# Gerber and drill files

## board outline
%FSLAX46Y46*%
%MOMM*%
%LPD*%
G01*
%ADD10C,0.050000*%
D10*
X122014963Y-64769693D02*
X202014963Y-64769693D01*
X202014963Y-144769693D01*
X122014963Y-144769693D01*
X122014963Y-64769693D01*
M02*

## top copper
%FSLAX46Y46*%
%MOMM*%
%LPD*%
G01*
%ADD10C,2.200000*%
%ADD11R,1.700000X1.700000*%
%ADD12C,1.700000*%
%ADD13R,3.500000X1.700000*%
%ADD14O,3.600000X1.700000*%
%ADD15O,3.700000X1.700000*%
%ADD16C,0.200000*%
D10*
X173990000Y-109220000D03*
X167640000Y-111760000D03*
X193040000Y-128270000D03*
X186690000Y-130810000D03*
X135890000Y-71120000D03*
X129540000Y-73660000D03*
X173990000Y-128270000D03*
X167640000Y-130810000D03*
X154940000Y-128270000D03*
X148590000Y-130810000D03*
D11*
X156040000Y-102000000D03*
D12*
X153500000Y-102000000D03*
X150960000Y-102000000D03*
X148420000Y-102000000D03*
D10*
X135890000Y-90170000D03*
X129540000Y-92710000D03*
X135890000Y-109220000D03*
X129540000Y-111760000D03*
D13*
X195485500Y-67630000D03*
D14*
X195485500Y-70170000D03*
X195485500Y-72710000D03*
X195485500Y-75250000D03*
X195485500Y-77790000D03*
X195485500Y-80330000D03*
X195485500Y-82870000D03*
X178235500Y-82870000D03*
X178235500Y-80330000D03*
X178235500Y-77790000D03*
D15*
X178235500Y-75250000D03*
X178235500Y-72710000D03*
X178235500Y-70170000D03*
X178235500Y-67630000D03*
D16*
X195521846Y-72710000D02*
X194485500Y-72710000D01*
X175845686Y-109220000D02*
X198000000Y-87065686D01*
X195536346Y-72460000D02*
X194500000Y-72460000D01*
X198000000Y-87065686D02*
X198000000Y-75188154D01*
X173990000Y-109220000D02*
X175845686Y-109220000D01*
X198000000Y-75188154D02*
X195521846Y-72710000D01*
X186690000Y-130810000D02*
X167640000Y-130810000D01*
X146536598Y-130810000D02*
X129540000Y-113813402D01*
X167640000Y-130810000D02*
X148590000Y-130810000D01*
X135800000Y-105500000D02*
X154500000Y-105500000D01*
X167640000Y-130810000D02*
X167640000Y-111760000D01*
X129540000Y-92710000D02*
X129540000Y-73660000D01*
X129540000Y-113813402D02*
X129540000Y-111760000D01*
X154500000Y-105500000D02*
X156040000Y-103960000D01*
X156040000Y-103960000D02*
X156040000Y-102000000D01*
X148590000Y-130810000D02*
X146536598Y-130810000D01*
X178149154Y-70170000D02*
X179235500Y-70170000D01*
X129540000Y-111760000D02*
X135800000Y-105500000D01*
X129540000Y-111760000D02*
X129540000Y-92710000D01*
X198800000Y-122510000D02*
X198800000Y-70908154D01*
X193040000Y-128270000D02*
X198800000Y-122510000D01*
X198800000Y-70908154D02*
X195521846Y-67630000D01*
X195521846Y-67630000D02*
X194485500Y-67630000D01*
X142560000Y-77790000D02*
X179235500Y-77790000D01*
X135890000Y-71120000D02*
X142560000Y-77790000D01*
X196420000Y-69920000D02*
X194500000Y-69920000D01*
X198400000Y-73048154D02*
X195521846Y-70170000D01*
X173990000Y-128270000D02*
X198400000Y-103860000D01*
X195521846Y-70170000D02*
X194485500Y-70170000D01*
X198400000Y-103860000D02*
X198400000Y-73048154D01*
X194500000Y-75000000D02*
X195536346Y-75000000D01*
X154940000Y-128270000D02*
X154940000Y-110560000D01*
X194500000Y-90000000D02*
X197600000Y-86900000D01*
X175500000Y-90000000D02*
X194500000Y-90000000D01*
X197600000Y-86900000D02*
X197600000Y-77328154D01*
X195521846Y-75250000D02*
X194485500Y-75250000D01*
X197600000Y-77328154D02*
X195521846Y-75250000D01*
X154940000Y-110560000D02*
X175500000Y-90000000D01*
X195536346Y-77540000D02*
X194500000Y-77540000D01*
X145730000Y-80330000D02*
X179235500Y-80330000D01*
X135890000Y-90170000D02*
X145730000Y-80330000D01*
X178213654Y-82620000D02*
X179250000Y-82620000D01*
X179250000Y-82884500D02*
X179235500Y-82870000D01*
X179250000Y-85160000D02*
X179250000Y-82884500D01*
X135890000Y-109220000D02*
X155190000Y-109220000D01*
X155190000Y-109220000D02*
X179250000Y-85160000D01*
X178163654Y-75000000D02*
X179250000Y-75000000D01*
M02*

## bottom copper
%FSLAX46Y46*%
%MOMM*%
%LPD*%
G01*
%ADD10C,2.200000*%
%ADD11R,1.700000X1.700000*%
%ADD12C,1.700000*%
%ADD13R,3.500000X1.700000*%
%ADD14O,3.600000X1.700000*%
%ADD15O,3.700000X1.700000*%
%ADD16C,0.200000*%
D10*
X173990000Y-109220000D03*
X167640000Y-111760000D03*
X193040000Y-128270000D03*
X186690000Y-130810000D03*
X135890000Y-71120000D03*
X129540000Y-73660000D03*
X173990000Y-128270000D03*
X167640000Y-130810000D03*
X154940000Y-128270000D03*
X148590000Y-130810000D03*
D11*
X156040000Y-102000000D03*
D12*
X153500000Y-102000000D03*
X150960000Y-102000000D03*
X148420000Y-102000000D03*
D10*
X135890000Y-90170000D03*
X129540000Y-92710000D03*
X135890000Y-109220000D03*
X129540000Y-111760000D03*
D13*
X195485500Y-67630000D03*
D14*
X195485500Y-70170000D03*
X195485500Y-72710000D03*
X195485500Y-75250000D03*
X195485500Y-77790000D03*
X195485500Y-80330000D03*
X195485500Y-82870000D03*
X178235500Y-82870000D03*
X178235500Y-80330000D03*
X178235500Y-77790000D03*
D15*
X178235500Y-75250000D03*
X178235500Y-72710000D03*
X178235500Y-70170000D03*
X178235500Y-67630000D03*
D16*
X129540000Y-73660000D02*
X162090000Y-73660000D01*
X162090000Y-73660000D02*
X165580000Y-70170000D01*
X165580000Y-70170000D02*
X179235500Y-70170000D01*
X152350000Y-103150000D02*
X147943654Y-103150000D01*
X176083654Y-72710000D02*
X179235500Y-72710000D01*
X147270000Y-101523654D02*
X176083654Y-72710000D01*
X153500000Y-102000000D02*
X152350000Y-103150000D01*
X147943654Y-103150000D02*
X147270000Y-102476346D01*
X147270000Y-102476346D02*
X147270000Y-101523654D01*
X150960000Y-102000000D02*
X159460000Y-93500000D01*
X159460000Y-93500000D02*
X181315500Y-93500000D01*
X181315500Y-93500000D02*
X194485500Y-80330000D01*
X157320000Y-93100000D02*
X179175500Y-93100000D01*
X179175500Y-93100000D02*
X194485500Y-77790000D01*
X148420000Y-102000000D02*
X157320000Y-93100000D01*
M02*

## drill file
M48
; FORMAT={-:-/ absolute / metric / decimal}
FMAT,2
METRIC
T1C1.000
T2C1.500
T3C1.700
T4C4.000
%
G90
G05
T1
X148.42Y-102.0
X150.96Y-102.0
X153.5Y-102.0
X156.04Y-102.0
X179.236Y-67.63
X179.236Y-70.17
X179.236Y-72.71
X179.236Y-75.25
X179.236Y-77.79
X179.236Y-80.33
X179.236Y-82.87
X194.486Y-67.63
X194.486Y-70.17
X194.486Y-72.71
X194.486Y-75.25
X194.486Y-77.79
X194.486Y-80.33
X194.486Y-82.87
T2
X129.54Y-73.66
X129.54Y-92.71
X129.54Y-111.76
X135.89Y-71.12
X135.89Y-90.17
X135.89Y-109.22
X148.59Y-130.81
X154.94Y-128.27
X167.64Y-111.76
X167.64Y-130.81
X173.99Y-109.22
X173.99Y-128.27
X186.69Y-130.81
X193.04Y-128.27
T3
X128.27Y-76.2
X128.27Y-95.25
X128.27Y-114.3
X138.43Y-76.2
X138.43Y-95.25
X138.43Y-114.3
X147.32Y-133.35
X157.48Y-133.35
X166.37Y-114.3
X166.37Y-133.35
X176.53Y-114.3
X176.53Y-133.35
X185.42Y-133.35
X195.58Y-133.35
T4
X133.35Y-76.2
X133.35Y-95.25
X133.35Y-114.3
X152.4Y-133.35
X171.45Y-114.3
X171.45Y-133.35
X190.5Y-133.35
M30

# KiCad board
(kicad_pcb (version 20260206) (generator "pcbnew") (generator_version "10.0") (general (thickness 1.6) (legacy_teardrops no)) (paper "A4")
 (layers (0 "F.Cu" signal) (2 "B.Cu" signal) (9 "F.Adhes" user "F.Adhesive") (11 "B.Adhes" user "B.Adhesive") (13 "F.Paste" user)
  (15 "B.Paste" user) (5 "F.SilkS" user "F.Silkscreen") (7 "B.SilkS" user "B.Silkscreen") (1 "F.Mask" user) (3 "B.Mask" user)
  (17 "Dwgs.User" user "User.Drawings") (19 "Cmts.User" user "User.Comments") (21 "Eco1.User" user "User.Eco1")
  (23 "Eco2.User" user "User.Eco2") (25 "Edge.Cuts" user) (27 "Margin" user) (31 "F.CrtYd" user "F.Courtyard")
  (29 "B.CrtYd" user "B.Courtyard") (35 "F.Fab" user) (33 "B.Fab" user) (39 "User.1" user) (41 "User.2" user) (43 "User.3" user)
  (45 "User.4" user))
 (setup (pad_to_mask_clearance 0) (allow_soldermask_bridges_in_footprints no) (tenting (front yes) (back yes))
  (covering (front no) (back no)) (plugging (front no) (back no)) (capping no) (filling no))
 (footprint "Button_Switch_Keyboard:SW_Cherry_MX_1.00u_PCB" (layer "F.Cu") (at 173.99 109.22)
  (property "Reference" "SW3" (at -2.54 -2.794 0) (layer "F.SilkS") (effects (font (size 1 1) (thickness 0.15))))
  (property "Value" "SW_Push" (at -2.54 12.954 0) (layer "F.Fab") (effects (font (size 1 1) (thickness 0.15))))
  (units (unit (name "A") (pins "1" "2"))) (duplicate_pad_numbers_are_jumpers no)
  (pad "" np_thru_hole circle (at -7.62 5.08) (size 1.7 1.7) (drill 1.7) (layers "*.Cu" "*.Mask"))
  (pad "" np_thru_hole circle (at -2.54 5.08) (size 4 4) (drill 4) (layers "*.Cu" "*.Mask"))
  (pad "" np_thru_hole circle (at 2.54 5.08) (size 1.7 1.7) (drill 1.7) (layers "*.Cu" "*.Mask"))
  (pad "1" thru_hole circle (at 0 0) (size 2.2 2.2) (drill 1.5) (layers "*.Cu" "*.Mask") (remove_unused_layers no)
   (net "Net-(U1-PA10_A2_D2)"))
  (pad "2" thru_hole circle (at -6.35 2.54) (size 2.2 2.2) (drill 1.5) (layers "*.Cu" "*.Mask") (remove_unused_layers no) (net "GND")))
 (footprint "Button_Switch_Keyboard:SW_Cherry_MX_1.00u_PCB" (layer "F.Cu") (at 193.04 128.27)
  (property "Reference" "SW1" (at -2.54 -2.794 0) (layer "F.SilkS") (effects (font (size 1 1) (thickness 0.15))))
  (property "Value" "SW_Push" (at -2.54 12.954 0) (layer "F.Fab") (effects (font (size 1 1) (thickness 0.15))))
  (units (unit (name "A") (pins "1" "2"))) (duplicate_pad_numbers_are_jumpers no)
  (pad "" np_thru_hole circle (at -7.62 5.08) (size 1.7 1.7) (drill 1.7) (layers "*.Cu" "*.Mask"))
  (pad "" np_thru_hole circle (at -2.54 5.08) (size 4 4) (drill 4) (layers "*.Cu" "*.Mask"))
  (pad "" np_thru_hole circle (at 2.54 5.08) (size 1.7 1.7) (drill 1.7) (layers "*.Cu" "*.Mask"))
  (pad "1" thru_hole circle (at 0 0) (size 2.2 2.2) (drill 1.5) (layers "*.Cu" "*.Mask") (remove_unused_layers no)
   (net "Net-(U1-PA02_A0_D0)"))
  (pad "2" thru_hole circle (at -6.35 2.54) (size 2.2 2.2) (drill 1.5) (layers "*.Cu" "*.Mask") (remove_unused_layers no) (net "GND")))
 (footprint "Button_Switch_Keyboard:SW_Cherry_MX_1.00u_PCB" (layer "F.Cu") (at 135.89 71.12)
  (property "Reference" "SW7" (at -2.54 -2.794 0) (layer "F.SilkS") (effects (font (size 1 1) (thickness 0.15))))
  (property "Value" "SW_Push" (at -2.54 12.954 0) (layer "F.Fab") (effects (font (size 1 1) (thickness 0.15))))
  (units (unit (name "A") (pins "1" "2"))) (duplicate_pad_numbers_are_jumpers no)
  (pad "" np_thru_hole circle (at -7.62 5.08) (size 1.7 1.7) (drill 1.7) (layers "*.Cu" "*.Mask"))
  (pad "" np_thru_hole circle (at -2.54 5.08) (size 4 4) (drill 4) (layers "*.Cu" "*.Mask"))
  (pad "" np_thru_hole circle (at 2.54 5.08) (size 1.7 1.7) (drill 1.7) (layers "*.Cu" "*.Mask"))
  (pad "1" thru_hole circle (at 0 0) (size 2.2 2.2) (drill 1.5) (layers "*.Cu" "*.Mask") (remove_unused_layers no)
   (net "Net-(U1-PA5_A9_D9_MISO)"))
  (pad "2" thru_hole circle (at -6.35 2.54) (size 2.2 2.2) (drill 1.5) (layers "*.Cu" "*.Mask") (remove_unused_layers no) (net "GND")))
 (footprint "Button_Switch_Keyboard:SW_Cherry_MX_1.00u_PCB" (layer "F.Cu") (at 173.99 128.27)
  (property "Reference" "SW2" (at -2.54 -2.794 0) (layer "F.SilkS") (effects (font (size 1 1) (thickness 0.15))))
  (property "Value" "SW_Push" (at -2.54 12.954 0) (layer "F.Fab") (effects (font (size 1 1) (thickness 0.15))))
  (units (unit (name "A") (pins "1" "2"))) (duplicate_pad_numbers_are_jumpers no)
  (pad "" np_thru_hole circle (at -7.62 5.08) (size 1.7 1.7) (drill 1.7) (layers "*.Cu" "*.Mask"))
  (pad "" np_thru_hole circle (at -2.54 5.08) (size 4 4) (drill 4) (layers "*.Cu" "*.Mask"))
  (pad "" np_thru_hole circle (at 2.54 5.08) (size 1.7 1.7) (drill 1.7) (layers "*.Cu" "*.Mask"))
  (pad "1" thru_hole circle (at 0 0) (size 2.2 2.2) (drill 1.5) (layers "*.Cu" "*.Mask") (remove_unused_layers no)
   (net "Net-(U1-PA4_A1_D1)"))
  (pad "2" thru_hole circle (at -6.35 2.54) (size 2.2 2.2) (drill 1.5) (layers "*.Cu" "*.Mask") (remove_unused_layers no) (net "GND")))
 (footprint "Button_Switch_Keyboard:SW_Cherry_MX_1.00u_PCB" (layer "F.Cu") (at 154.94 128.27)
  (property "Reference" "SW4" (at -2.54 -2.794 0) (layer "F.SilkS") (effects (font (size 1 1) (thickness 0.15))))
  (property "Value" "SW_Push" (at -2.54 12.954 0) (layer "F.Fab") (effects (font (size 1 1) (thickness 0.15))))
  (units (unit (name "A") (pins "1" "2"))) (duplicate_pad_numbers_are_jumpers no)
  (pad "" np_thru_hole circle (at -7.62 5.08) (size 1.7 1.7) (drill 1.7) (layers "*.Cu" "*.Mask"))
  (pad "" np_thru_hole circle (at -2.54 5.08) (size 4 4) (drill 4) (layers "*.Cu" "*.Mask"))
  (pad "" np_thru_hole circle (at 2.54 5.08) (size 1.7 1.7) (drill 1.7) (layers "*.Cu" "*.Mask"))
  (pad "1" thru_hole circle (at 0 0) (size 2.2 2.2) (drill 1.5) (layers "*.Cu" "*.Mask") (remove_unused_layers no)
   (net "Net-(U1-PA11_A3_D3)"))
  (pad "2" thru_hole circle (at -6.35 2.54) (size 2.2 2.2) (drill 1.5) (layers "*.Cu" "*.Mask") (remove_unused_layers no) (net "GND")))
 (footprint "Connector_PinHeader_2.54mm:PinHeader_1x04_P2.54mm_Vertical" (layer "F.Cu") (at 156.04 102 -90)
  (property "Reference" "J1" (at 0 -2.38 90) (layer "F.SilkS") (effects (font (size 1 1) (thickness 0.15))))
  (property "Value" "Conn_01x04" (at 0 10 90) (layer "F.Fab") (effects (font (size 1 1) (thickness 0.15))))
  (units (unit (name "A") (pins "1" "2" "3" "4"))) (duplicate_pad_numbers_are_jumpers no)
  (pad "1" thru_hole rect (at 0 0 270) (size 1.7 1.7) (drill 1) (layers "*.Cu" "*.Mask") (remove_unused_layers no) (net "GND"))
  (pad "2" thru_hole circle (at 0 2.54 270) (size 1.7 1.7) (drill 1) (layers "*.Cu" "*.Mask") (remove_unused_layers no) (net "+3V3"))
  (pad "3" thru_hole circle (at 0 5.08 270) (size 1.7 1.7) (drill 1) (layers "*.Cu" "*.Mask") (remove_unused_layers no)
   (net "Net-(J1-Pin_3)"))
  (pad "4" thru_hole circle (at 0 7.62 270) (size 1.7 1.7) (drill 1) (layers "*.Cu" "*.Mask") (remove_unused_layers no)
   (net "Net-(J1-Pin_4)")))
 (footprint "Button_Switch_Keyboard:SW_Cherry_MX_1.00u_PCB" (layer "F.Cu") (at 135.89 90.17)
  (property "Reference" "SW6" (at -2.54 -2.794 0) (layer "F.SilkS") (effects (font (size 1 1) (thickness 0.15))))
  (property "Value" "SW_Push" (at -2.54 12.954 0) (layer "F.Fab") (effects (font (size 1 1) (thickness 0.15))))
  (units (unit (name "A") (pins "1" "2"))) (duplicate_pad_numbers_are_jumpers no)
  (pad "" np_thru_hole circle (at -7.62 5.08) (size 1.7 1.7) (drill 1.7) (layers "*.Cu" "*.Mask"))
  (pad "" np_thru_hole circle (at -2.54 5.08) (size 4 4) (drill 4) (layers "*.Cu" "*.Mask"))
  (pad "" np_thru_hole circle (at 2.54 5.08) (size 1.7 1.7) (drill 1.7) (layers "*.Cu" "*.Mask"))
  (pad "1" thru_hole circle (at 0 0) (size 2.2 2.2) (drill 1.5) (layers "*.Cu" "*.Mask") (remove_unused_layers no)
   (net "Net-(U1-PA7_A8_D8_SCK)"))
  (pad "2" thru_hole circle (at -6.35 2.54) (size 2.2 2.2) (drill 1.5) (layers "*.Cu" "*.Mask") (remove_unused_layers no) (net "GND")))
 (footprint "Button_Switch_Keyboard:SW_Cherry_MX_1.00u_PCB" (layer "F.Cu") (at 135.89 109.22)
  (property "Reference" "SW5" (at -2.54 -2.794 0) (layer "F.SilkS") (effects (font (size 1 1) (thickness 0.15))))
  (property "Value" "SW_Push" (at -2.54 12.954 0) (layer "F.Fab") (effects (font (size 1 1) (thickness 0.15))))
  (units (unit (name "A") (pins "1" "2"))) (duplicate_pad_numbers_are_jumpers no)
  (pad "" np_thru_hole circle (at -7.62 5.08) (size 1.7 1.7) (drill 1.7) (layers "*.Cu" "*.Mask"))
  (pad "" np_thru_hole circle (at -2.54 5.08) (size 4 4) (drill 4) (layers "*.Cu" "*.Mask"))
  (pad "" np_thru_hole circle (at 2.54 5.08) (size 1.7 1.7) (drill 1.7) (layers "*.Cu" "*.Mask"))
  (pad "1" thru_hole circle (at 0 0) (size 2.2 2.2) (drill 1.5) (layers "*.Cu" "*.Mask") (remove_unused_layers no)
   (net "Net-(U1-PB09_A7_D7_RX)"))
  (pad "2" thru_hole circle (at -6.35 2.54) (size 2.2 2.2) (drill 1.5) (layers "*.Cu" "*.Mask") (remove_unused_layers no) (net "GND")))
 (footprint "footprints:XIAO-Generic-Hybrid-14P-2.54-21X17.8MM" (layer "B.Cu") (at 186.8605 75.25 180)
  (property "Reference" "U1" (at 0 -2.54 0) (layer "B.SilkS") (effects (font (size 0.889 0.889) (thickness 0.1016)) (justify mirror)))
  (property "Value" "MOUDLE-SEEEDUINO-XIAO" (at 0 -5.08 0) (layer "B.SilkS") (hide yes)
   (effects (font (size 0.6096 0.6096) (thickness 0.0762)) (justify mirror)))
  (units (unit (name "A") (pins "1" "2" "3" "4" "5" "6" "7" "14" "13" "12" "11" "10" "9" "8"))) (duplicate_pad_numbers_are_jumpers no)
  (pad "1" thru_hole rect (at -7.625 7.62 180) (size 3.5 1.7) (drill 1 (offset -1 0)) (layers "*.Cu" "*.Mask") (remove_unused_layers no)
   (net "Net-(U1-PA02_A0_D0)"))
  (pad "2" thru_hole oval (at -7.625 5.08 180) (size 3.6 1.7) (drill 1 (offset -1 0)) (layers "*.Cu" "*.Mask") (remove_unused_layers no)
   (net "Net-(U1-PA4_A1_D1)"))
  (pad "3" thru_hole oval (at -7.625 2.54 180) (size 3.6 1.7) (drill 1 (offset -1 0)) (layers "*.Cu" "*.Mask") (remove_unused_layers no)
   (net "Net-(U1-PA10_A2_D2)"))
  (pad "4" thru_hole oval (at -7.625 0 180) (size 3.6 1.7) (drill 1 (offset -1 0)) (layers "*.Cu" "*.Mask") (remove_unused_layers no)
   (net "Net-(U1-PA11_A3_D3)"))
  (pad "5" thru_hole oval (at -7.625 -2.54 180) (size 3.6 1.7) (drill 1 (offset -1 0)) (layers "*.Cu" "*.Mask") (remove_unused_layers no)
   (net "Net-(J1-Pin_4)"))
  (pad "6" thru_hole oval (at -7.625 -5.08) (size 3.6 1.7) (drill 1 (offset 1 0)) (layers "*.Cu" "*.Mask") (remove_unused_layers no)
   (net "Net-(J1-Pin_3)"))
  (pad "7" thru_hole oval (at -7.625 -7.62 180) (size 3.6 1.7) (drill 1 (offset -1 0)) (layers "*.Cu" "*.Mask") (remove_unused_layers no)
   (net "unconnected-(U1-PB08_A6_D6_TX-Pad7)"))
  (pad "8" thru_hole oval (at 7.625 -7.62 180) (size 3.6 1.7) (drill 1 (offset 1 0)) (layers "*.Cu" "*.Mask") (remove_unused_layers no)
   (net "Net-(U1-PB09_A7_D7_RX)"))
  (pad "9" thru_hole oval (at 7.625 -5.08 180) (size 3.6 1.7) (drill 1 (offset 1 0)) (layers "*.Cu" "*.Mask") (remove_unused_layers no)
   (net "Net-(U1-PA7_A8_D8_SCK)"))
  (pad "10" thru_hole oval (at 7.625 -2.54 180) (size 3.6 1.7) (drill 1 (offset 1 0)) (layers "*.Cu" "*.Mask") (remove_unused_layers no)
   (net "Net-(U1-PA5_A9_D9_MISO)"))
  (pad "11" thru_hole oval (at 7.625 0 180) (size 3.7 1.7) (drill 1 (offset 1 0)) (layers "*.Cu" "*.Mask") (remove_unused_layers no)
   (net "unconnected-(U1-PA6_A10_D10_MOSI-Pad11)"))
  (pad "12" thru_hole oval (at 7.625 2.54 180) (size 3.7 1.7) (drill 1 (offset 1 0)) (layers "*.Cu" "*.Mask") (remove_unused_layers no)
   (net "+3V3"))
  (pad "13" thru_hole oval (at 7.625 5.08 180) (size 3.7 1.7) (drill 1 (offset 1 0)) (layers "*.Cu" "*.Mask") (remove_unused_layers no)
   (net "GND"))
  (pad "14" thru_hole oval (at 7.625 7.62 180) (size 3.7 1.7) (drill 1 (offset 1 0)) (layers "*.Cu" "*.Mask") (remove_unused_layers no)
   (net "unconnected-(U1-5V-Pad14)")))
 (gr_rect (start 122.014963 64.769693) (end 202.014963 144.769693) (stroke (width 0.05) (type solid)) (fill no) (layer "Edge.Cuts"))
 (segment (start 195.521846 72.71) (end 194.4855 72.71) (width 0.2) (layer "F.Cu") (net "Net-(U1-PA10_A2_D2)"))
 (segment (start 175.845686 109.22) (end 198 87.065686) (width 0.2) (layer "F.Cu") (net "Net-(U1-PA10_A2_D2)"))
 (segment (start 195.536346 72.46) (end 194.5 72.46) (width 0.2) (layer "F.Cu") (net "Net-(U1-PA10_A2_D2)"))
 (segment (start 198 87.065686) (end 198 75.188154) (width 0.2) (layer "F.Cu") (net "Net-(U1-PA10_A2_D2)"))
 (segment (start 173.99 109.22) (end 175.845686 109.22) (width 0.2) (layer "F.Cu") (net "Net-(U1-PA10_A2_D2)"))
 (segment (start 198 75.188154) (end 195.521846 72.71) (width 0.2) (layer "F.Cu") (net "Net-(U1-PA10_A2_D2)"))
 (segment (start 186.69 130.81) (end 167.64 130.81) (width 0.2) (layer "F.Cu") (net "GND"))
 (segment (start 146.536598 130.81) (end 129.54 113.813402) (width 0.2) (layer "F.Cu") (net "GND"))
 (segment (start 167.64 130.81) (end 148.59 130.81) (width 0.2) (layer "F.Cu") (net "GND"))
 (segment (start 135.8 105.5) (end 154.5 105.5) (width 0.2) (layer "F.Cu") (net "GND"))
 (segment (start 167.64 130.81) (end 167.64 111.76) (width 0.2) (layer "F.Cu") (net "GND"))
 (segment (start 129.54 92.71) (end 129.54 73.66) (width 0.2) (layer "F.Cu") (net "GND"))
 (segment (start 129.54 113.813402) (end 129.54 111.76) (width 0.2) (layer "F.Cu") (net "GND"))
 (segment (start 154.5 105.5) (end 156.04 103.96) (width 0.2) (layer "F.Cu") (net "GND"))
 (segment (start 156.04 103.96) (end 156.04 102) (width 0.2) (layer "F.Cu") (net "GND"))
 (segment (start 148.59 130.81) (end 146.536598 130.81) (width 0.2) (layer "F.Cu") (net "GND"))
 (segment (start 178.149154 70.17) (end 179.2355 70.17) (width 0.2) (layer "F.Cu") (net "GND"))
 (segment (start 129.54 111.76) (end 135.8 105.5) (width 0.2) (layer "F.Cu") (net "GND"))
 (segment (start 129.54 111.76) (end 129.54 92.71) (width 0.2) (layer "F.Cu") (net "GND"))
 (segment (start 129.54 73.66) (end 162.09 73.66) (width 0.2) (layer "B.Cu") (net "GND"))
 (segment (start 162.09 73.66) (end 165.58 70.17) (width 0.2) (layer "B.Cu") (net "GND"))
 (segment (start 165.58 70.17) (end 179.2355 70.17) (width 0.2) (layer "B.Cu") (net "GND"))
 (segment (start 198.8 122.51) (end 198.8 70.908154) (width 0.2) (layer "F.Cu") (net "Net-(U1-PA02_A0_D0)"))
 (segment (start 193.04 128.27) (end 198.8 122.51) (width 0.2) (layer "F.Cu") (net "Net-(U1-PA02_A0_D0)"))
 (segment (start 198.8 70.908154) (end 195.521846 67.63) (width 0.2) (layer "F.Cu") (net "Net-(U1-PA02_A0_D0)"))
 (segment (start 195.521846 67.63) (end 194.4855 67.63) (width 0.2) (layer "F.Cu") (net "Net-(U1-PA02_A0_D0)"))
 (segment (start 142.56 77.79) (end 179.2355 77.79) (width 0.2) (layer "F.Cu") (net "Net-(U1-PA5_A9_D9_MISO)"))
 (segment (start 135.89 71.12) (end 142.56 77.79) (width 0.2) (layer "F.Cu") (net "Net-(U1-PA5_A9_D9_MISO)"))
 (segment (start 196.42 69.92) (end 194.5 69.92) (width 0.2) (layer "F.Cu") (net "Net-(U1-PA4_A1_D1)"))
 (segment (start 198.4 73.048154) (end 195.521846 70.17) (width 0.2) (layer "F.Cu") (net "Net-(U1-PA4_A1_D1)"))
 (segment (start 173.99 128.27) (end 198.4 103.86) (width 0.2) (layer "F.Cu") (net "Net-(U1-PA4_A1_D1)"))
 (segment (start 195.521846 70.17) (end 194.4855 70.17) (width 0.2) (layer "F.Cu") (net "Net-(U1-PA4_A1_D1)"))
 (segment (start 198.4 103.86) (end 198.4 73.048154) (width 0.2) (layer "F.Cu") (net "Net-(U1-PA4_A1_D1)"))
 (segment (start 194.5 75) (end 195.536346 75) (width 0.2) (layer "F.Cu") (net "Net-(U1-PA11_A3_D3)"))
 (segment (start 154.94 128.27) (end 154.94 110.56) (width 0.2) (layer "F.Cu") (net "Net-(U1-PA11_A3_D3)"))
 (segment (start 194.5 90) (end 197.6 86.9) (width 0.2) (layer "F.Cu") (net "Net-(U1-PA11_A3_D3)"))
 (segment (start 175.5 90) (end 194.5 90) (width 0.2) (layer "F.Cu") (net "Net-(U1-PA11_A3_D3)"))
 (segment (start 197.6 86.9) (end 197.6 77.328154) (width 0.2) (layer "F.Cu") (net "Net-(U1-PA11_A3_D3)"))
 (segment (start 195.521846 75.25) (end 194.4855 75.25) (width 0.2) (layer "F.Cu") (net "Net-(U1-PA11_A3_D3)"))
 (segment (start 197.6 77.328154) (end 195.521846 75.25) (width 0.2) (layer "F.Cu") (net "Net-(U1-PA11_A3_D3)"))
 (segment (start 154.94 110.56) (end 175.5 90) (width 0.2) (layer "F.Cu") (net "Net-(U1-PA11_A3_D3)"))
 (segment (start 152.35 103.15) (end 147.943654 103.15) (width 0.2) (layer "B.Cu") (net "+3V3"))
 (segment (start 176.083654 72.71) (end 179.2355 72.71) (width 0.2) (layer "B.Cu") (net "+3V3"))
 (segment (start 147.27 101.523654) (end 176.083654 72.71) (width 0.2) (layer "B.Cu") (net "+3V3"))
 (segment (start 153.5 102) (end 152.35 103.15) (width 0.2) (layer "B.Cu") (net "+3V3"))
 (segment (start 147.943654 103.15) (end 147.27 102.476346) (width 0.2) (layer "B.Cu") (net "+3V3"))
 (segment (start 147.27 102.476346) (end 147.27 101.523654) (width 0.2) (layer "B.Cu") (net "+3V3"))
 (segment (start 150.96 102) (end 159.46 93.5) (width 0.2) (layer "B.Cu") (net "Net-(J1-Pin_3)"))
 (segment (start 159.46 93.5) (end 181.3155 93.5) (width 0.2) (layer "B.Cu") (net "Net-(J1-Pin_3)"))
 (segment (start 181.3155 93.5) (end 194.4855 80.33) (width 0.2) (layer "B.Cu") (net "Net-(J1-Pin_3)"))
 (segment (start 195.536346 77.54) (end 194.5 77.54) (width 0.2) (layer "F.Cu") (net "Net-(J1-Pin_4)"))
 (segment (start 157.32 93.1) (end 179.1755 93.1) (width 0.2) (layer "B.Cu") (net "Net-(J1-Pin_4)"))
 (segment (start 179.1755 93.1) (end 194.4855 77.79) (width 0.2) (layer "B.Cu") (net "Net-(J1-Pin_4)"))
 (segment (start 148.42 102) (end 157.32 93.1) (width 0.2) (layer "B.Cu") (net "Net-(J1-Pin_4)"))
 (segment (start 145.73 80.33) (end 179.2355 80.33) (width 0.2) (layer "F.Cu") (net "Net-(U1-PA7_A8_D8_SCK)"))
 (segment (start 135.89 90.17) (end 145.73 80.33) (width 0.2) (layer "F.Cu") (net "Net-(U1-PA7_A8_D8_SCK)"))
 (segment (start 178.213654 82.62) (end 179.25 82.62) (width 0.2) (layer "F.Cu") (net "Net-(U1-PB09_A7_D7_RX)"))
 (segment (start 179.25 82.8845) (end 179.2355 82.87) (width 0.2) (layer "F.Cu") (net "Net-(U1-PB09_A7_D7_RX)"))
 (segment (start 179.25 85.16) (end 179.25 82.8845) (width 0.2) (layer "F.Cu") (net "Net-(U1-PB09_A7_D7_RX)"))
 (segment (start 135.89 109.22) (end 155.19 109.22) (width 0.2) (layer "F.Cu") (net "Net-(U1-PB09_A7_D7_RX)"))
 (segment (start 155.19 109.22) (end 179.25 85.16) (width 0.2) (layer "F.Cu") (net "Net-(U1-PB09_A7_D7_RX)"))
 (segment (start 178.163654 75) (end 179.25 75) (width 0.2) (layer "F.Cu") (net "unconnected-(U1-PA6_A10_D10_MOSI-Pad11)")))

